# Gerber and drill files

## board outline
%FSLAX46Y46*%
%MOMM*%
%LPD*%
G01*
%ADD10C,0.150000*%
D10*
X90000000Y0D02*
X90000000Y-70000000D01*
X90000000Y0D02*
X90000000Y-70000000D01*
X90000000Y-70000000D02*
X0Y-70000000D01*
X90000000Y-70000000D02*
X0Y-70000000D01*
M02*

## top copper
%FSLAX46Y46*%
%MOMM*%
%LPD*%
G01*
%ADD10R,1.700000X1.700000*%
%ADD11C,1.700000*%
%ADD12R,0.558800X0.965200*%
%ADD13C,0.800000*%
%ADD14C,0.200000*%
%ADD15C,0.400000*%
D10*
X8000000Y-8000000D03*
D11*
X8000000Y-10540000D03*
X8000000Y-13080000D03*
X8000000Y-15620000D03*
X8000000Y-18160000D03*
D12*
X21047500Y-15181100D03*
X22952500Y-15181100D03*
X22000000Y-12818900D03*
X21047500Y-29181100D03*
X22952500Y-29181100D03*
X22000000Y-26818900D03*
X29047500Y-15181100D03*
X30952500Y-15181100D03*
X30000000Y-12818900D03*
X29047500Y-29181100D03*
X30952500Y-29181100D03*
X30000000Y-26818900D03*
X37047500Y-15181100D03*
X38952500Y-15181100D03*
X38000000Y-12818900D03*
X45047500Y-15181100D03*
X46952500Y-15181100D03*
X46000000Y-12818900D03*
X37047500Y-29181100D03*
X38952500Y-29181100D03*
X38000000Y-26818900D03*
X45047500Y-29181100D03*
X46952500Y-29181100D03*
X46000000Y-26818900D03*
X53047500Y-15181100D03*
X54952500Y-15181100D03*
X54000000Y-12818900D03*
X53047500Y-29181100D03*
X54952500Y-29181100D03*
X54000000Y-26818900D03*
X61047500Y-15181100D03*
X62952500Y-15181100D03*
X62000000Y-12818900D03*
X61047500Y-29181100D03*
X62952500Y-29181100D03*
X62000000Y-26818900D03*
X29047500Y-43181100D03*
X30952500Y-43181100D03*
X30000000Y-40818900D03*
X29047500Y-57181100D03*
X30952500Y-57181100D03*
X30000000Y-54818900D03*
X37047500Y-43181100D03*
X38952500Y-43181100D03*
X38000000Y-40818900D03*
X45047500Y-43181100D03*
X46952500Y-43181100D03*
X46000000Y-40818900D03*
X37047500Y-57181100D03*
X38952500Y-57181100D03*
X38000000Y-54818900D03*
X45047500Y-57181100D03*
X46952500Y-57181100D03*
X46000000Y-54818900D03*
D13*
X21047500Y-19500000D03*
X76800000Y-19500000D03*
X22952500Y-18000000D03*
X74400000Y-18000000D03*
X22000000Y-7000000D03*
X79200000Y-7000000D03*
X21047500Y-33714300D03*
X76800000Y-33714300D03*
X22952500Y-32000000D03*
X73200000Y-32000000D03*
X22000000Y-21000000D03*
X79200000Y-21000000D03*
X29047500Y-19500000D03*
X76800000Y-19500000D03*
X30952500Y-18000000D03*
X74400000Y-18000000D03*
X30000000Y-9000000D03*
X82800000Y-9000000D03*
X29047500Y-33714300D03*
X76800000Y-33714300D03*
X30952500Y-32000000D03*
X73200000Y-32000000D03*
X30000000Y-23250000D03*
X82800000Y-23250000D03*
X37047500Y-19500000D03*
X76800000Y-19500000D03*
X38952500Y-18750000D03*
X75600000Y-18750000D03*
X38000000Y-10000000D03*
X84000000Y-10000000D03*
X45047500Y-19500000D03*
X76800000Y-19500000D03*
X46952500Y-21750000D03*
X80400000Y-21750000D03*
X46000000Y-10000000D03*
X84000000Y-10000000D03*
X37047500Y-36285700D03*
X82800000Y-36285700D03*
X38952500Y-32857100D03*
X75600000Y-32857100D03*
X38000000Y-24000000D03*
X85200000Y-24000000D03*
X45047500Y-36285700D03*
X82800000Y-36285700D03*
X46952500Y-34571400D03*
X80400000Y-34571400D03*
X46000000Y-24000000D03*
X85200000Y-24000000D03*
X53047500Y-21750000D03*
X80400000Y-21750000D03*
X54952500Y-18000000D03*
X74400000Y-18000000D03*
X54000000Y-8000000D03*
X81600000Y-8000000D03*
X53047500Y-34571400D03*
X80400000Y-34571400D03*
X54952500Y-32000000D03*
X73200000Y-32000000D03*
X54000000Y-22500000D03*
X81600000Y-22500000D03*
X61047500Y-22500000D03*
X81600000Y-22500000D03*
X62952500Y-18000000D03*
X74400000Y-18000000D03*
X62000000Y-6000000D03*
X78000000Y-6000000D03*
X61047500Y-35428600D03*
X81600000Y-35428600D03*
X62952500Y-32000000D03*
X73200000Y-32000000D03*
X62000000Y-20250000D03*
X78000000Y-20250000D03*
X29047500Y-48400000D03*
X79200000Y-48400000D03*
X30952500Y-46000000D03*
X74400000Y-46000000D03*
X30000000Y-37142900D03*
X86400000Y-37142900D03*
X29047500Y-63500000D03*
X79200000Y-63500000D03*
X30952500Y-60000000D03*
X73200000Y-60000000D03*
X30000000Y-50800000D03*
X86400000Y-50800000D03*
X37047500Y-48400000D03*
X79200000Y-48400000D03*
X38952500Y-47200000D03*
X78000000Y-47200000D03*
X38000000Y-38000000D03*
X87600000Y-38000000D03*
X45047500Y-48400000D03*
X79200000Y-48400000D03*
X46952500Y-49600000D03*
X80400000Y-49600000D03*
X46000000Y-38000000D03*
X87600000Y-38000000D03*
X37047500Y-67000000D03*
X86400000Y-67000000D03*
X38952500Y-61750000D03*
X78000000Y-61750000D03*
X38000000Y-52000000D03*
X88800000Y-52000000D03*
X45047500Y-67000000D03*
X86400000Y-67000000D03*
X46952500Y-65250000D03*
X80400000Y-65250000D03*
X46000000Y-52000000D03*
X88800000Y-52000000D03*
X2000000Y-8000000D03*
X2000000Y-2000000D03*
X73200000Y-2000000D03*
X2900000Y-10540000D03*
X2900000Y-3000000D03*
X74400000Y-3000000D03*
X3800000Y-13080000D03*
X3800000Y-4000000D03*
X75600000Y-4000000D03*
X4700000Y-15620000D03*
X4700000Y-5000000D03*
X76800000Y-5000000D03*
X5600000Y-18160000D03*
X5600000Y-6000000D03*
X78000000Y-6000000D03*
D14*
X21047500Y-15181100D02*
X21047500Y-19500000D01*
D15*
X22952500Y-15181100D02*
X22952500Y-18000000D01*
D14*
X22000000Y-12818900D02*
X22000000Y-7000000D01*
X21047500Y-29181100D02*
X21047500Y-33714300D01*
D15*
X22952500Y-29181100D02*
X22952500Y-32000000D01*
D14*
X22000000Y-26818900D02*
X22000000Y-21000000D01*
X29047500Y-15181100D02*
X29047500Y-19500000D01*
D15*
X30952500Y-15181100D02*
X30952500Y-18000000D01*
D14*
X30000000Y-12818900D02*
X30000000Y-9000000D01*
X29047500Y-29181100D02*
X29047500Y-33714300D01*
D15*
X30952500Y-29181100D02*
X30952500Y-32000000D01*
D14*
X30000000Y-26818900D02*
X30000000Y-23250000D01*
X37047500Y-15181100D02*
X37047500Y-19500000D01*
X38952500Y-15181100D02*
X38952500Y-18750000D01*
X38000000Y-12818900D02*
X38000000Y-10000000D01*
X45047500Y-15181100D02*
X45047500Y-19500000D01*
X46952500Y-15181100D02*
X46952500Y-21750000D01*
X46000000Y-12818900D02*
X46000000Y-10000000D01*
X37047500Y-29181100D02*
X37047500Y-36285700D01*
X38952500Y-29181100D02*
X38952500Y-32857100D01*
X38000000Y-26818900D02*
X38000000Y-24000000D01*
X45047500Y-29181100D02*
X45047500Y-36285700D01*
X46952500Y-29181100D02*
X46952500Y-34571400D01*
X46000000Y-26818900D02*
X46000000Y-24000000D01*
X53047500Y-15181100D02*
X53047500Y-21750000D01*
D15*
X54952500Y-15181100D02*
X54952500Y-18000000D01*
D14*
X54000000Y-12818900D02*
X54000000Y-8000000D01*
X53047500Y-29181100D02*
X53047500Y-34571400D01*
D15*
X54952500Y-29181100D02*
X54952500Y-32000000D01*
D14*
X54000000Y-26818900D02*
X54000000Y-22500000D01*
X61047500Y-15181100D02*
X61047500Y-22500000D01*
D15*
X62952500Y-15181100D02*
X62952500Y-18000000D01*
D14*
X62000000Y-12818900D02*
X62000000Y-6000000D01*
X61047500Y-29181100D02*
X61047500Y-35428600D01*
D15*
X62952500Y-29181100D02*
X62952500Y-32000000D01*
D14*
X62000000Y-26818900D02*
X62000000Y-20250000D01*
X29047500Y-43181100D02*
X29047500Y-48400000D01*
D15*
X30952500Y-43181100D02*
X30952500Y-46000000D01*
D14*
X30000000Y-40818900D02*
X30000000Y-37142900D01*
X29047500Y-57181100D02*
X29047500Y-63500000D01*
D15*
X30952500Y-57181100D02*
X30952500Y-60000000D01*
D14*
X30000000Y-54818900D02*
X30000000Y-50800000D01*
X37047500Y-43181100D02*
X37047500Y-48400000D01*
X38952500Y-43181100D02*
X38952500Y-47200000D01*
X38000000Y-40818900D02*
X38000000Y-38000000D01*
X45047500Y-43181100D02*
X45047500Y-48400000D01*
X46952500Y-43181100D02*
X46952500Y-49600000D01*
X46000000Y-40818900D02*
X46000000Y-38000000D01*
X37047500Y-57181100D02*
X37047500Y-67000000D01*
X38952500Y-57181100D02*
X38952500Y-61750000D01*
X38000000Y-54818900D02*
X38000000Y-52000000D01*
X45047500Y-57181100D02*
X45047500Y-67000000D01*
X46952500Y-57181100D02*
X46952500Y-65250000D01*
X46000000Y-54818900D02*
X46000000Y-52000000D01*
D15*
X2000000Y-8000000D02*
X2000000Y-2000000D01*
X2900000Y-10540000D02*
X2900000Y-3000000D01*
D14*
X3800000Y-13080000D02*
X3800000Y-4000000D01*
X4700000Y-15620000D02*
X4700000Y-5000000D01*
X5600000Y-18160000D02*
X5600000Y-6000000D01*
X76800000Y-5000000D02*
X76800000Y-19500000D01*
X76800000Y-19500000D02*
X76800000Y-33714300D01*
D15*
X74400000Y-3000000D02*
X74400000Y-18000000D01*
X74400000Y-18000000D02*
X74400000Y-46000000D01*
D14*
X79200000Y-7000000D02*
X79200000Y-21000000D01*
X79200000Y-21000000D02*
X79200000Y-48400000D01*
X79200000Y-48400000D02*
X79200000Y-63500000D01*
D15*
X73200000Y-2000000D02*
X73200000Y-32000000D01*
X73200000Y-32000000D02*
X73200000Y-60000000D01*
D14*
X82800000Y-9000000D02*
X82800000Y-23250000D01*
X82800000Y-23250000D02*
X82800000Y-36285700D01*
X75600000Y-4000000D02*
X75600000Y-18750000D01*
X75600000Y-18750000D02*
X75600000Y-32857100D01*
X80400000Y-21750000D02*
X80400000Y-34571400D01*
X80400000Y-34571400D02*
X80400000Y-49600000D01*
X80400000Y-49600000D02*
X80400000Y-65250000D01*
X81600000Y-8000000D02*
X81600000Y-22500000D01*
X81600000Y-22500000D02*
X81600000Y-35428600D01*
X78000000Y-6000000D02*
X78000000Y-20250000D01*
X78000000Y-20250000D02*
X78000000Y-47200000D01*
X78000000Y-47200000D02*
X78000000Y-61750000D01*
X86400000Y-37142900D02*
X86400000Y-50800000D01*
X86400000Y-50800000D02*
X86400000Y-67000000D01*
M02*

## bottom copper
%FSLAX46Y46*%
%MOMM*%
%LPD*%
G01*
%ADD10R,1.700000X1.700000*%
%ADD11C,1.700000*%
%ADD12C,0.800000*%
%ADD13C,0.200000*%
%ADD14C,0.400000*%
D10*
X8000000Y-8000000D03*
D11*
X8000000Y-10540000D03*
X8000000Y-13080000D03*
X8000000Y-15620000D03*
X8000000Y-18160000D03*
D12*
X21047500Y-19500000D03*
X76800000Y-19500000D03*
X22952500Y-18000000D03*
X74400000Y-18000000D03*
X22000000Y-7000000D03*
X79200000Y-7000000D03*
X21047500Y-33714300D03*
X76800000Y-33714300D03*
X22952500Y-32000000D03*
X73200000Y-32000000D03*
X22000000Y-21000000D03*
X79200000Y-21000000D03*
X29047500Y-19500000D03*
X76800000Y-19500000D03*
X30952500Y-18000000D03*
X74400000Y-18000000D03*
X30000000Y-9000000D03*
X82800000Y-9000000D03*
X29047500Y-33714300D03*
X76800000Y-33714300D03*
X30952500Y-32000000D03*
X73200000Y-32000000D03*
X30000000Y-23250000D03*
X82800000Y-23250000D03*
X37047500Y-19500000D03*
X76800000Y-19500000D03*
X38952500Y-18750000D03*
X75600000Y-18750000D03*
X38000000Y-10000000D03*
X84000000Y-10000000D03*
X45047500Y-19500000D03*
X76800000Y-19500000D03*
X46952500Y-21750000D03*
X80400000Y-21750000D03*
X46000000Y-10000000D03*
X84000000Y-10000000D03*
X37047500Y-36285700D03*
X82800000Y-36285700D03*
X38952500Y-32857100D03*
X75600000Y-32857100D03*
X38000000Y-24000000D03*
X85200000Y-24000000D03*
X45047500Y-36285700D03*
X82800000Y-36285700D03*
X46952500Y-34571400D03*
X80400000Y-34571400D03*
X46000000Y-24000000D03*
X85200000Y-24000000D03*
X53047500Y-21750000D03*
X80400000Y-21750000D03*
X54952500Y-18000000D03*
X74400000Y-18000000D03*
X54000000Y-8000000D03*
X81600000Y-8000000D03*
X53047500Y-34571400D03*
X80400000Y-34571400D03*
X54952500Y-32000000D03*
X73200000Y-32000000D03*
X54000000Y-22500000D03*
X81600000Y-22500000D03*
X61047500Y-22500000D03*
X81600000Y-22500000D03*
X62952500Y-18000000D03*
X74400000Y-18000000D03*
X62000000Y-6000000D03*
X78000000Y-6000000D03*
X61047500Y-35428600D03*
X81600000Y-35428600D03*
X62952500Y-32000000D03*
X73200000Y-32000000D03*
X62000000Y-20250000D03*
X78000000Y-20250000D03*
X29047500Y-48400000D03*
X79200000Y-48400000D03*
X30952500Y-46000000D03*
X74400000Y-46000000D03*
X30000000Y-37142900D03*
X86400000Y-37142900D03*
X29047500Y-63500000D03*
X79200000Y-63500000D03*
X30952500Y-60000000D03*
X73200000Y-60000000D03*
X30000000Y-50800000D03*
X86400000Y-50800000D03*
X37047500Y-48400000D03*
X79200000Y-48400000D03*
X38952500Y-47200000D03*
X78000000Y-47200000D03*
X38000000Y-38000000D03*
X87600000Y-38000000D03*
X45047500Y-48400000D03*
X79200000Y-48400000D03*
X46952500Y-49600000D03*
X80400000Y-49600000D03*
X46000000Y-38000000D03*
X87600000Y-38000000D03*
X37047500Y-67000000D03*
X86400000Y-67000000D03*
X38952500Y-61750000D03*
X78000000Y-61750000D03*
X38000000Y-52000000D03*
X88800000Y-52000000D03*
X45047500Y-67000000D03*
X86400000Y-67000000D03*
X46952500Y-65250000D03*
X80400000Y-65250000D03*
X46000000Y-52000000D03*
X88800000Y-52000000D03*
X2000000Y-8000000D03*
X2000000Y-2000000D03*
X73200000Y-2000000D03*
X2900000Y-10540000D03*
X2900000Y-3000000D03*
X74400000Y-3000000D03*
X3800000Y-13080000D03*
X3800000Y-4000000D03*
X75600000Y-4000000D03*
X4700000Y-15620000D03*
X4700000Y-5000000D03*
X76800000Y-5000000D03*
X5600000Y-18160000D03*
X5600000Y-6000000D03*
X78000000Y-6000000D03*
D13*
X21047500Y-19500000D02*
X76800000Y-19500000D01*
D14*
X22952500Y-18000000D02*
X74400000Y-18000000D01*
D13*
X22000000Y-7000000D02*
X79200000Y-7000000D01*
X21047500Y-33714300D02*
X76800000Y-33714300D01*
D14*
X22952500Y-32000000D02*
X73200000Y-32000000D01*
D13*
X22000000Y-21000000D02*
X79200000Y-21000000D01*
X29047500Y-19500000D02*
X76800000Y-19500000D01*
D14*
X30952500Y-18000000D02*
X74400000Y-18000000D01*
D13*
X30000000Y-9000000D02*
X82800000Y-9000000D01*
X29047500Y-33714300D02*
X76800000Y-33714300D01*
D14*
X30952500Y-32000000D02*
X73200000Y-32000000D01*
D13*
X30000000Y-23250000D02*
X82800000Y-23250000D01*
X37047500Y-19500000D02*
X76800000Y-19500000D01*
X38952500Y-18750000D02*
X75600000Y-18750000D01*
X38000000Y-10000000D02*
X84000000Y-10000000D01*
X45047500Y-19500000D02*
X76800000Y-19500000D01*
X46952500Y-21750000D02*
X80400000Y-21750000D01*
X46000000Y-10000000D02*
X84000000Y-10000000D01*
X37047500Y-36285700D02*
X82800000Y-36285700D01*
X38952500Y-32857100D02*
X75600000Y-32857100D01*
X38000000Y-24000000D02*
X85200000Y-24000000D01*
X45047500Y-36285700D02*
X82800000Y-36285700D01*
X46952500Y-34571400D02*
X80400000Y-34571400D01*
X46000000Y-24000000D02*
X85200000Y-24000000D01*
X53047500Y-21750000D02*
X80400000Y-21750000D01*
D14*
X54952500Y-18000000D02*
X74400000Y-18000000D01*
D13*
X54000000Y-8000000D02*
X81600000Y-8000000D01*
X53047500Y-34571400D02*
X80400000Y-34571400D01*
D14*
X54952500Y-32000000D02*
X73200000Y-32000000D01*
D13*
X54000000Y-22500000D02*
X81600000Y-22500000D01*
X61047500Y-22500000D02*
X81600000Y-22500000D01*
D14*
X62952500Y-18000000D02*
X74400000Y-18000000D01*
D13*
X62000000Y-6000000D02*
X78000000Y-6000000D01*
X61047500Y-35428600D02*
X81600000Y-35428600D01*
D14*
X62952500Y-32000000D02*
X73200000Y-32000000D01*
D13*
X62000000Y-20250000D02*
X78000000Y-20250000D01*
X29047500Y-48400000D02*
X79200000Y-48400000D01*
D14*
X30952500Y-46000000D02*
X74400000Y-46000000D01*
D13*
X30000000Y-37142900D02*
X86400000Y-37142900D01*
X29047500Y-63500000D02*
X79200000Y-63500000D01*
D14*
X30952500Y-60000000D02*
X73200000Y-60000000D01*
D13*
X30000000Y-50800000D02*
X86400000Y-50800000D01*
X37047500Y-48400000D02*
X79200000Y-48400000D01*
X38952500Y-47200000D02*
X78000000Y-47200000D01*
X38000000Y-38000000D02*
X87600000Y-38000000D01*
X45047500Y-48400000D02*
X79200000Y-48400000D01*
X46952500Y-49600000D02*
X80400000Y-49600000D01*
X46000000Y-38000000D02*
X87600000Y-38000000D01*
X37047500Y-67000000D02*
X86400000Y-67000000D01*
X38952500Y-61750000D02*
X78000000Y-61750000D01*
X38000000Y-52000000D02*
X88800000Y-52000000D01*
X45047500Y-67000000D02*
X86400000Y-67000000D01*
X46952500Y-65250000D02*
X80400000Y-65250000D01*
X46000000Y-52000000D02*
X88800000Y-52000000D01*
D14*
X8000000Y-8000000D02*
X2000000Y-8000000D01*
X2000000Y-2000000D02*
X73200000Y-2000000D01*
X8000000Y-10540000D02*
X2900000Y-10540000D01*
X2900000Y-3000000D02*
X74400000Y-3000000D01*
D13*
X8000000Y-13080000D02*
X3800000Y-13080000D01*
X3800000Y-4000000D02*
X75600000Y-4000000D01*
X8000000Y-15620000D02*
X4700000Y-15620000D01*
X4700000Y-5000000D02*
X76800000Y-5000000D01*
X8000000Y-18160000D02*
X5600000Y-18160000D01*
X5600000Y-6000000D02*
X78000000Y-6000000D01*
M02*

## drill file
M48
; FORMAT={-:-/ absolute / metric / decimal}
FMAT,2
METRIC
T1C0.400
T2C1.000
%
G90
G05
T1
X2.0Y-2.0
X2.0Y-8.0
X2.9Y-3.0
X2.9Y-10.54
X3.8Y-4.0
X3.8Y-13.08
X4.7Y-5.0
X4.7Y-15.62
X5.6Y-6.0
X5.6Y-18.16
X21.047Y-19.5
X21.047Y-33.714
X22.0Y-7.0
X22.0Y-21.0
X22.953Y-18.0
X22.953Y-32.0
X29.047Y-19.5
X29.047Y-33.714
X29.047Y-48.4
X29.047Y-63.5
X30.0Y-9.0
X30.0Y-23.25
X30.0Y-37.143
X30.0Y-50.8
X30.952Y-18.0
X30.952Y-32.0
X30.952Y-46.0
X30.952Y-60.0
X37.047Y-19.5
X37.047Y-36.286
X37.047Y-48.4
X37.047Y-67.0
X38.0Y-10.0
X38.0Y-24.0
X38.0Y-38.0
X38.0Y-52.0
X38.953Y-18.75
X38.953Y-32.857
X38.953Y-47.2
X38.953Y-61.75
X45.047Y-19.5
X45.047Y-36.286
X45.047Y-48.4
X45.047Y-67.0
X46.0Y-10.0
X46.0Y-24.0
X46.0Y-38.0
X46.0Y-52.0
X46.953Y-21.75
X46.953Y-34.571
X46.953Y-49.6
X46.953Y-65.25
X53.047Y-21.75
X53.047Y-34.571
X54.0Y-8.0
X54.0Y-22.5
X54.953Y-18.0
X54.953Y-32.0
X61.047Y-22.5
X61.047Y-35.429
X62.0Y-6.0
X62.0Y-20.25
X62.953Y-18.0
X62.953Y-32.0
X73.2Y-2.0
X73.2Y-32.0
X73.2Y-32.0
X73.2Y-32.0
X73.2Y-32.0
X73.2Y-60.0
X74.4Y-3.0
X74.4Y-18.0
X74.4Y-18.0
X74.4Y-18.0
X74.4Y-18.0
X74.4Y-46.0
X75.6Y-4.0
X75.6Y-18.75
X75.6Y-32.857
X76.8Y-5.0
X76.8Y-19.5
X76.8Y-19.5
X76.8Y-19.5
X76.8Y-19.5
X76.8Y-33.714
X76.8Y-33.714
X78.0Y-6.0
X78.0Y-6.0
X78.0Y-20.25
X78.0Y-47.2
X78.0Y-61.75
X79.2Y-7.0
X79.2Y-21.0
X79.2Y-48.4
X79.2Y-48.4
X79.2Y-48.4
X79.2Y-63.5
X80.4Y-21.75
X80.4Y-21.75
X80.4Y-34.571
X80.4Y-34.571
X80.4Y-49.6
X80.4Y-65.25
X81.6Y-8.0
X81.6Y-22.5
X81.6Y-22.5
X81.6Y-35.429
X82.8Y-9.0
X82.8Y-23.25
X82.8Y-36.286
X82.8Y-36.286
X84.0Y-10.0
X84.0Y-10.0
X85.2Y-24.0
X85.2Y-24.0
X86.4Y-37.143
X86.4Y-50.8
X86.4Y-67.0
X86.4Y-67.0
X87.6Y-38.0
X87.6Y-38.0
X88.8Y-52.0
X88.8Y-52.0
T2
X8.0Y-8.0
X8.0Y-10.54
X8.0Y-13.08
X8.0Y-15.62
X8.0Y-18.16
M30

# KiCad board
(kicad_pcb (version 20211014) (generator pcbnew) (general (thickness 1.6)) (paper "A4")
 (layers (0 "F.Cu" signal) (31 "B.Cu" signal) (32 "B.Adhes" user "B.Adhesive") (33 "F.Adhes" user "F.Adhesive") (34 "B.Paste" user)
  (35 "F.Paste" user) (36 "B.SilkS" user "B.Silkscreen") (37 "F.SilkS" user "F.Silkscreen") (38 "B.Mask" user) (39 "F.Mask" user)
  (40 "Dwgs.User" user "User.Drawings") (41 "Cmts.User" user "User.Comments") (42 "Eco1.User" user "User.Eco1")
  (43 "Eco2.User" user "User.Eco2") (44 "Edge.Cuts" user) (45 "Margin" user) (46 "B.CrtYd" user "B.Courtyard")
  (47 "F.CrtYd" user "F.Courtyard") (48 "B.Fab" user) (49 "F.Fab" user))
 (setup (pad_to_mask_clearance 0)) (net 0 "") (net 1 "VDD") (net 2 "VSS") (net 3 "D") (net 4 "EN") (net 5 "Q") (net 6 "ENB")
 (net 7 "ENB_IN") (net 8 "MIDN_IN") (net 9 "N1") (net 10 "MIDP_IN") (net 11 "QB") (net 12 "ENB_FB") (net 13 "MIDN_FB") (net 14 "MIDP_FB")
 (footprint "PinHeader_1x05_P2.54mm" (layer "F.Cu") (at 8.0 8.0)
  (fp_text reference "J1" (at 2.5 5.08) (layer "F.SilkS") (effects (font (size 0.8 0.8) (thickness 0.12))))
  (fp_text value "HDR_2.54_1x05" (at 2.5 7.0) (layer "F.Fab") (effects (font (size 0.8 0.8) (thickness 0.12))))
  (pad "1" thru_hole rect (at 0 0.0) (size 1.7 1.7) (drill 1.0) (layers *.Cu *.Mask) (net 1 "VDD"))
  (pad "2" thru_hole circle (at 0 2.54) (size 1.7 1.7) (drill 1.0) (layers *.Cu *.Mask) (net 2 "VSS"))
  (pad "3" thru_hole circle (at 0 5.08) (size 1.7 1.7) (drill 1.0) (layers *.Cu *.Mask) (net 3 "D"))
  (pad "4" thru_hole circle (at 0 7.62) (size 1.7 1.7) (drill 1.0) (layers *.Cu *.Mask) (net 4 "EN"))
  (pad "5" thru_hole circle (at 0 10.16) (size 1.7 1.7) (drill 1.0) (layers *.Cu *.Mask) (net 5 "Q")))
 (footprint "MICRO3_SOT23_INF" (layer "F.Cu") (at 22.0000 14.0000)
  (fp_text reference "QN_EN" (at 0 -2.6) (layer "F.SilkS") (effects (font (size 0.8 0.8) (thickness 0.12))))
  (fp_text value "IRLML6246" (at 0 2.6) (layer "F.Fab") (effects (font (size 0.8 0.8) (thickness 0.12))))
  (pad "1" smd rect (at -0.9525 1.1811) (size 0.5588 0.9652) (layers "F.Cu" "F.Paste" "F.Mask") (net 4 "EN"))
  (pad "2" smd rect (at 0.9525 1.1811) (size 0.5588 0.9652) (layers "F.Cu" "F.Paste" "F.Mask") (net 2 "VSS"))
  (pad "3" smd rect (at 0 -1.1811) (size 0.5588 0.9652) (layers "F.Cu" "F.Paste" "F.Mask") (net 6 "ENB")))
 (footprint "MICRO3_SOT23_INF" (layer "F.Cu") (at 22.0000 28.0000)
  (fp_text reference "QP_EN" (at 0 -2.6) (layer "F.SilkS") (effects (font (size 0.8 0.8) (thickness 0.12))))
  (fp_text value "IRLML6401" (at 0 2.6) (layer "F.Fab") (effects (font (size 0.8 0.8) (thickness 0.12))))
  (pad "1" smd rect (at -0.9525 1.1811) (size 0.5588 0.9652) (layers "F.Cu" "F.Paste" "F.Mask") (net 4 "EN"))
  (pad "2" smd rect (at 0.9525 1.1811) (size 0.5588 0.9652) (layers "F.Cu" "F.Paste" "F.Mask") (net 1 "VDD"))
  (pad "3" smd rect (at 0 -1.1811) (size 0.5588 0.9652) (layers "F.Cu" "F.Paste" "F.Mask") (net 6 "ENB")))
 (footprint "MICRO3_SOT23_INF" (layer "F.Cu") (at 30.0000 14.0000)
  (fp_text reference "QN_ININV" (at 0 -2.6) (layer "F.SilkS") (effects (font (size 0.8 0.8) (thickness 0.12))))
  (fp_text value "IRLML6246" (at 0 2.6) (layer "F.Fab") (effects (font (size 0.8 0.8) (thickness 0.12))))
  (pad "1" smd rect (at -0.9525 1.1811) (size 0.5588 0.9652) (layers "F.Cu" "F.Paste" "F.Mask") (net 4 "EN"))
  (pad "2" smd rect (at 0.9525 1.1811) (size 0.5588 0.9652) (layers "F.Cu" "F.Paste" "F.Mask") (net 2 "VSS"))
  (pad "3" smd rect (at 0 -1.1811) (size 0.5588 0.9652) (layers "F.Cu" "F.Paste" "F.Mask") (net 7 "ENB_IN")))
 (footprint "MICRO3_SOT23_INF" (layer "F.Cu") (at 30.0000 28.0000)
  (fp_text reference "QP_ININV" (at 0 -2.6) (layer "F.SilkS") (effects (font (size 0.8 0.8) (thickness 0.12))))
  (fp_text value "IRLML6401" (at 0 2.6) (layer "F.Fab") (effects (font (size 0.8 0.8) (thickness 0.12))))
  (pad "1" smd rect (at -0.9525 1.1811) (size 0.5588 0.9652) (layers "F.Cu" "F.Paste" "F.Mask") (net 4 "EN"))
  (pad "2" smd rect (at 0.9525 1.1811) (size 0.5588 0.9652) (layers "F.Cu" "F.Paste" "F.Mask") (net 1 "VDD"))
  (pad "3" smd rect (at 0 -1.1811) (size 0.5588 0.9652) (layers "F.Cu" "F.Paste" "F.Mask") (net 7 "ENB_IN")))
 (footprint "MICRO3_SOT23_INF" (layer "F.Cu") (at 38.0000 14.0000)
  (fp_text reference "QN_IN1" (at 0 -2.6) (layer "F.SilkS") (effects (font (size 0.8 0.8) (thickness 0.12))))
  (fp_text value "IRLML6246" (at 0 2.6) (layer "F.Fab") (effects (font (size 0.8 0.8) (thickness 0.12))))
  (pad "1" smd rect (at -0.9525 1.1811) (size 0.5588 0.9652) (layers "F.Cu" "F.Paste" "F.Mask") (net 4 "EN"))
  (pad "2" smd rect (at 0.9525 1.1811) (size 0.5588 0.9652) (layers "F.Cu" "F.Paste" "F.Mask") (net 3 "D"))
  (pad "3" smd rect (at 0 -1.1811) (size 0.5588 0.9652) (layers "F.Cu" "F.Paste" "F.Mask") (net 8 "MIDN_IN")))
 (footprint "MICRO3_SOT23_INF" (layer "F.Cu") (at 46.0000 14.0000)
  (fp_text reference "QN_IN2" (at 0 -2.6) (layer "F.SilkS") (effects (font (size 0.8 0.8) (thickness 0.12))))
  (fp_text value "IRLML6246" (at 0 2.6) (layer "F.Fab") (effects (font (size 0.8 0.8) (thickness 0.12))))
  (pad "1" smd rect (at -0.9525 1.1811) (size 0.5588 0.9652) (layers "F.Cu" "F.Paste" "F.Mask") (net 4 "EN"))
  (pad "2" smd rect (at 0.9525 1.1811) (size 0.5588 0.9652) (layers "F.Cu" "F.Paste" "F.Mask") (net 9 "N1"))
  (pad "3" smd rect (at 0 -1.1811) (size 0.5588 0.9652) (layers "F.Cu" "F.Paste" "F.Mask") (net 8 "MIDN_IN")))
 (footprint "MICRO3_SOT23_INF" (layer "F.Cu") (at 38.0000 28.0000)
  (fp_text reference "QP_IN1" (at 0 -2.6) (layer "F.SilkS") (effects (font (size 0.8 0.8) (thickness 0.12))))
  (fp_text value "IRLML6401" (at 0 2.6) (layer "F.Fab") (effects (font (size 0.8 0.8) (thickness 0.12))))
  (pad "1" smd rect (at -0.9525 1.1811) (size 0.5588 0.9652) (layers "F.Cu" "F.Paste" "F.Mask") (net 7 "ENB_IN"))
  (pad "2" smd rect (at 0.9525 1.1811) (size 0.5588 0.9652) (layers "F.Cu" "F.Paste" "F.Mask") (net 3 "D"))
  (pad "3" smd rect (at 0 -1.1811) (size 0.5588 0.9652) (layers "F.Cu" "F.Paste" "F.Mask") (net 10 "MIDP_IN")))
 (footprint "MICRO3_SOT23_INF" (layer "F.Cu") (at 46.0000 28.0000)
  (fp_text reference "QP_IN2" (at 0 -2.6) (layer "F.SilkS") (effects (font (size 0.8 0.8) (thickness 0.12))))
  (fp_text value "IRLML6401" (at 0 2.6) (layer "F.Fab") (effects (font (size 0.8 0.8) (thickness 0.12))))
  (pad "1" smd rect (at -0.9525 1.1811) (size 0.5588 0.9652) (layers "F.Cu" "F.Paste" "F.Mask") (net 7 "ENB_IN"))
  (pad "2" smd rect (at 0.9525 1.1811) (size 0.5588 0.9652) (layers "F.Cu" "F.Paste" "F.Mask") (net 9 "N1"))
  (pad "3" smd rect (at 0 -1.1811) (size 0.5588 0.9652) (layers "F.Cu" "F.Paste" "F.Mask") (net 10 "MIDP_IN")))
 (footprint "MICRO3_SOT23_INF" (layer "F.Cu") (at 54.0000 14.0000)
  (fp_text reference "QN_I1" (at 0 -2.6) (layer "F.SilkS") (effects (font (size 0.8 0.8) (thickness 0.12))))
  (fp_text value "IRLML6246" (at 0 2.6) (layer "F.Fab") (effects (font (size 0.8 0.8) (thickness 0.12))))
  (pad "1" smd rect (at -0.9525 1.1811) (size 0.5588 0.9652) (layers "F.Cu" "F.Paste" "F.Mask") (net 9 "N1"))
  (pad "2" smd rect (at 0.9525 1.1811) (size 0.5588 0.9652) (layers "F.Cu" "F.Paste" "F.Mask") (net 2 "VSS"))
  (pad "3" smd rect (at 0 -1.1811) (size 0.5588 0.9652) (layers "F.Cu" "F.Paste" "F.Mask") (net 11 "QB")))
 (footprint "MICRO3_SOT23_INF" (layer "F.Cu") (at 54.0000 28.0000)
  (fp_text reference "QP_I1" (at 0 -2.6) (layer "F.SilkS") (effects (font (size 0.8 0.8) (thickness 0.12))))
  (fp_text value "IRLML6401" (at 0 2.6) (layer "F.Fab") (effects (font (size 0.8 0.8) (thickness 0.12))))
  (pad "1" smd rect (at -0.9525 1.1811) (size 0.5588 0.9652) (layers "F.Cu" "F.Paste" "F.Mask") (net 9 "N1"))
  (pad "2" smd rect (at 0.9525 1.1811) (size 0.5588 0.9652) (layers "F.Cu" "F.Paste" "F.Mask") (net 1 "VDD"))
  (pad "3" smd rect (at 0 -1.1811) (size 0.5588 0.9652) (layers "F.Cu" "F.Paste" "F.Mask") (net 11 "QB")))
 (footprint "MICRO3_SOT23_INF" (layer "F.Cu") (at 62.0000 14.0000)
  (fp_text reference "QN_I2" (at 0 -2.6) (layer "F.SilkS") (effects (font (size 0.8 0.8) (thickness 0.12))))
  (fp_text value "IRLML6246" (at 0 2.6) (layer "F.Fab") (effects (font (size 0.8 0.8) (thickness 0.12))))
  (pad "1" smd rect (at -0.9525 1.1811) (size 0.5588 0.9652) (layers "F.Cu" "F.Paste" "F.Mask") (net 11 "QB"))
  (pad "2" smd rect (at 0.9525 1.1811) (size 0.5588 0.9652) (layers "F.Cu" "F.Paste" "F.Mask") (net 2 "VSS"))
  (pad "3" smd rect (at 0 -1.1811) (size 0.5588 0.9652) (layers "F.Cu" "F.Paste" "F.Mask") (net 5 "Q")))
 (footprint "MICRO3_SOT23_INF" (layer "F.Cu") (at 62.0000 28.0000)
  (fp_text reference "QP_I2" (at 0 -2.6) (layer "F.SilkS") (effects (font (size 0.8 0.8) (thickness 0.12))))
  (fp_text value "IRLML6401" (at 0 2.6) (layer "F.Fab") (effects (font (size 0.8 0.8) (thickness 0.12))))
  (pad "1" smd rect (at -0.9525 1.1811) (size 0.5588 0.9652) (layers "F.Cu" "F.Paste" "F.Mask") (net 11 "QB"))
  (pad "2" smd rect (at 0.9525 1.1811) (size 0.5588 0.9652) (layers "F.Cu" "F.Paste" "F.Mask") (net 1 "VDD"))
  (pad "3" smd rect (at 0 -1.1811) (size 0.5588 0.9652) (layers "F.Cu" "F.Paste" "F.Mask") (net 5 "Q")))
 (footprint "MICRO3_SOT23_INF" (layer "F.Cu") (at 30.0000 42.0000)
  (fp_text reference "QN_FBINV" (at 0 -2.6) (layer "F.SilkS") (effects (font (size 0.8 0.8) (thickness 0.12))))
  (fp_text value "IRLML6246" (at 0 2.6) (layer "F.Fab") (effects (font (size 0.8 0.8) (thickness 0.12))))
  (pad "1" smd rect (at -0.9525 1.1811) (size 0.5588 0.9652) (layers "F.Cu" "F.Paste" "F.Mask") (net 6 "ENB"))
  (pad "2" smd rect (at 0.9525 1.1811) (size 0.5588 0.9652) (layers "F.Cu" "F.Paste" "F.Mask") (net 2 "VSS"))
  (pad "3" smd rect (at 0 -1.1811) (size 0.5588 0.9652) (layers "F.Cu" "F.Paste" "F.Mask") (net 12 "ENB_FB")))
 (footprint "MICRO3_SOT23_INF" (layer "F.Cu") (at 30.0000 56.0000)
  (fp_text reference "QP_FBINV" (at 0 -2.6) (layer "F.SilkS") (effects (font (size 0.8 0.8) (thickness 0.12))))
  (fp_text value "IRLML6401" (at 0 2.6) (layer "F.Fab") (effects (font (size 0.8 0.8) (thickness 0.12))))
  (pad "1" smd rect (at -0.9525 1.1811) (size 0.5588 0.9652) (layers "F.Cu" "F.Paste" "F.Mask") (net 6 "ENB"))
  (pad "2" smd rect (at 0.9525 1.1811) (size 0.5588 0.9652) (layers "F.Cu" "F.Paste" "F.Mask") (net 1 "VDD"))
  (pad "3" smd rect (at 0 -1.1811) (size 0.5588 0.9652) (layers "F.Cu" "F.Paste" "F.Mask") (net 12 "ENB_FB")))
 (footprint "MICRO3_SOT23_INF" (layer "F.Cu") (at 38.0000 42.0000)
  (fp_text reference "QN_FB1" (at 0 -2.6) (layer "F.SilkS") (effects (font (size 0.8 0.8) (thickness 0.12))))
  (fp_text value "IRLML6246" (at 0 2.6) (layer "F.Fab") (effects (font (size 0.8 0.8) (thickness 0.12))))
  (pad "1" smd rect (at -0.9525 1.1811) (size 0.5588 0.9652) (layers "F.Cu" "F.Paste" "F.Mask") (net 6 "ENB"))
  (pad "2" smd rect (at 0.9525 1.1811) (size 0.5588 0.9652) (layers "F.Cu" "F.Paste" "F.Mask") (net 5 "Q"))
  (pad "3" smd rect (at 0 -1.1811) (size 0.5588 0.9652) (layers "F.Cu" "F.Paste" "F.Mask") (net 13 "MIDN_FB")))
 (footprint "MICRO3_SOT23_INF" (layer "F.Cu") (at 46.0000 42.0000)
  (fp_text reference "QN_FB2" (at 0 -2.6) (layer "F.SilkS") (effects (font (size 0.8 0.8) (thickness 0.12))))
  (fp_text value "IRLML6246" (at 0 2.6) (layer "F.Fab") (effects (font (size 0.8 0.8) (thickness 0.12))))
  (pad "1" smd rect (at -0.9525 1.1811) (size 0.5588 0.9652) (layers "F.Cu" "F.Paste" "F.Mask") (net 6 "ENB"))
  (pad "2" smd rect (at 0.9525 1.1811) (size 0.5588 0.9652) (layers "F.Cu" "F.Paste" "F.Mask") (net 9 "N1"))
  (pad "3" smd rect (at 0 -1.1811) (size 0.5588 0.9652) (layers "F.Cu" "F.Paste" "F.Mask") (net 13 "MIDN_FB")))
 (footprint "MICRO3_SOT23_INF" (layer "F.Cu") (at 38.0000 56.0000)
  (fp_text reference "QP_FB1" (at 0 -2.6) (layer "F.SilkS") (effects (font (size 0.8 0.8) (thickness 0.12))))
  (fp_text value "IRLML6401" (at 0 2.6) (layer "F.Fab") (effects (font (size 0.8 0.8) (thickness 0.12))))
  (pad "1" smd rect (at -0.9525 1.1811) (size 0.5588 0.9652) (layers "F.Cu" "F.Paste" "F.Mask") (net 12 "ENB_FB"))
  (pad "2" smd rect (at 0.9525 1.1811) (size 0.5588 0.9652) (layers "F.Cu" "F.Paste" "F.Mask") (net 5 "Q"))
  (pad "3" smd rect (at 0 -1.1811) (size 0.5588 0.9652) (layers "F.Cu" "F.Paste" "F.Mask") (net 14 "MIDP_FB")))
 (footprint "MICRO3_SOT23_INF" (layer "F.Cu") (at 46.0000 56.0000)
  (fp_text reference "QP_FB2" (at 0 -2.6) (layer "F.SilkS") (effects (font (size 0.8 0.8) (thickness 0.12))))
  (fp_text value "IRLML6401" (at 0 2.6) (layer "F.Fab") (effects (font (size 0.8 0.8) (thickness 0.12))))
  (pad "1" smd rect (at -0.9525 1.1811) (size 0.5588 0.9652) (layers "F.Cu" "F.Paste" "F.Mask") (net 12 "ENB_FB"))
  (pad "2" smd rect (at 0.9525 1.1811) (size 0.5588 0.9652) (layers "F.Cu" "F.Paste" "F.Mask") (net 9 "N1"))
  (pad "3" smd rect (at 0 -1.1811) (size 0.5588 0.9652) (layers "F.Cu" "F.Paste" "F.Mask") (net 14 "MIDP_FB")))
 (gr_line (start 90 0) (end 90 70) (layer "Edge.Cuts") (width 0.15))
 (gr_line (start 90 0) (end 90 70) (layer "Edge.Cuts") (width 0.15))
 (gr_line (start 90 70) (end 0 70) (layer "Edge.Cuts") (width 0.15))
 (gr_line (start 90 70) (end 0 70) (layer "Edge.Cuts") (width 0.15))
 (segment (start 21.0475 15.1811) (end 21.0475 19.5) (width 0.2) (layer "F.Cu") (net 4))
 (segment (start 21.0475 19.5) (end 76.8 19.5) (width 0.2) (layer "B.Cu") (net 4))
 (segment (start 22.9525 15.1811) (end 22.9525 18.0) (width 0.4) (layer "F.Cu") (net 2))
 (segment (start 22.9525 18.0) (end 74.4 18.0) (width 0.4) (layer "B.Cu") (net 2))
 (segment (start 22.0 12.8189) (end 22.0 7.0) (width 0.2) (layer "F.Cu") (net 6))
 (segment (start 22.0 7.0) (end 79.2 7.0) (width 0.2) (layer "B.Cu") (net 6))
 (segment (start 21.0475 29.1811) (end 21.0475 33.7143) (width 0.2) (layer "F.Cu") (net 4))
 (segment (start 21.0475 33.7143) (end 76.8 33.7143) (width 0.2) (layer "B.Cu") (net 4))
 (segment (start 22.9525 29.1811) (end 22.9525 32.0) (width 0.4) (layer "F.Cu") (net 1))
 (segment (start 22.9525 32.0) (end 73.2 32.0) (width 0.4) (layer "B.Cu") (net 1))
 (segment (start 22.0 26.8189) (end 22.0 21.0) (width 0.2) (layer "F.Cu") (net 6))
 (segment (start 22.0 21.0) (end 79.2 21.0) (width 0.2) (layer "B.Cu") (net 6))
 (segment (start 29.0475 15.1811) (end 29.0475 19.5) (width 0.2) (layer "F.Cu") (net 4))
 (segment (start 29.0475 19.5) (end 76.8 19.5) (width 0.2) (layer "B.Cu") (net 4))
 (segment (start 30.9525 15.1811) (end 30.9525 18.0) (width 0.4) (layer "F.Cu") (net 2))
 (segment (start 30.9525 18.0) (end 74.4 18.0) (width 0.4) (layer "B.Cu") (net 2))
 (segment (start 30.0 12.8189) (end 30.0 9.0) (width 0.2) (layer "F.Cu") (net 7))
 (segment (start 30.0 9.0) (end 82.8 9.0) (width 0.2) (layer "B.Cu") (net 7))
 (segment (start 29.0475 29.1811) (end 29.0475 33.7143) (width 0.2) (layer "F.Cu") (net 4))
 (segment (start 29.0475 33.7143) (end 76.8 33.7143) (width 0.2) (layer "B.Cu") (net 4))
 (segment (start 30.9525 29.1811) (end 30.9525 32.0) (width 0.4) (layer "F.Cu") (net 1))
 (segment (start 30.9525 32.0) (end 73.2 32.0) (width 0.4) (layer "B.Cu") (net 1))
 (segment (start 30.0 26.8189) (end 30.0 23.25) (width 0.2) (layer "F.Cu") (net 7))
 (segment (start 30.0 23.25) (end 82.8 23.25) (width 0.2) (layer "B.Cu") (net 7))
 (segment (start 37.0475 15.1811) (end 37.0475 19.5) (width 0.2) (layer "F.Cu") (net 4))
 (segment (start 37.0475 19.5) (end 76.8 19.5) (width 0.2) (layer "B.Cu") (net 4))
 (segment (start 38.9525 15.1811) (end 38.9525 18.75) (width 0.2) (layer "F.Cu") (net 3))
 (segment (start 38.9525 18.75) (end 75.6 18.75) (width 0.2) (layer "B.Cu") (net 3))
 (segment (start 38.0 12.8189) (end 38.0 10.0) (width 0.2) (layer "F.Cu") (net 8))
 (segment (start 38.0 10.0) (end 84.0 10.0) (width 0.2) (layer "B.Cu") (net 8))
 (segment (start 45.0475 15.1811) (end 45.0475 19.5) (width 0.2) (layer "F.Cu") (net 4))
 (segment (start 45.0475 19.5) (end 76.8 19.5) (width 0.2) (layer "B.Cu") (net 4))
 (segment (start 46.9525 15.1811) (end 46.9525 21.75) (width 0.2) (layer "F.Cu") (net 9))
 (segment (start 46.9525 21.75) (end 80.4 21.75) (width 0.2) (layer "B.Cu") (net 9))
 (segment (start 46.0 12.8189) (end 46.0 10.0) (width 0.2) (layer "F.Cu") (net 8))
 (segment (start 46.0 10.0) (end 84.0 10.0) (width 0.2) (layer "B.Cu") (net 8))
 (segment (start 37.0475 29.1811) (end 37.0475 36.2857) (width 0.2) (layer "F.Cu") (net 7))
 (segment (start 37.0475 36.2857) (end 82.8 36.2857) (width 0.2) (layer "B.Cu") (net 7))
 (segment (start 38.9525 29.1811) (end 38.9525 32.8571) (width 0.2) (layer "F.Cu") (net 3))
 (segment (start 38.9525 32.8571) (end 75.6 32.8571) (width 0.2) (layer "B.Cu") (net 3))
 (segment (start 38.0 26.8189) (end 38.0 24.0) (width 0.2) (layer "F.Cu") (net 10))
 (segment (start 38.0 24.0) (end 85.2 24.0) (width 0.2) (layer "B.Cu") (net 10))
 (segment (start 45.0475 29.1811) (end 45.0475 36.2857) (width 0.2) (layer "F.Cu") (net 7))
 (segment (start 45.0475 36.2857) (end 82.8 36.2857) (width 0.2) (layer "B.Cu") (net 7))
 (segment (start 46.9525 29.1811) (end 46.9525 34.5714) (width 0.2) (layer "F.Cu") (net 9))
 (segment (start 46.9525 34.5714) (end 80.4 34.5714) (width 0.2) (layer "B.Cu") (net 9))
 (segment (start 46.0 26.8189) (end 46.0 24.0) (width 0.2) (layer "F.Cu") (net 10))
 (segment (start 46.0 24.0) (end 85.2 24.0) (width 0.2) (layer "B.Cu") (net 10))
 (segment (start 53.0475 15.1811) (end 53.0475 21.75) (width 0.2) (layer "F.Cu") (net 9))
 (segment (start 53.0475 21.75) (end 80.4 21.75) (width 0.2) (layer "B.Cu") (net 9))
 (segment (start 54.9525 15.1811) (end 54.9525 18.0) (width 0.4) (layer "F.Cu") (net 2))
 (segment (start 54.9525 18.0) (end 74.4 18.0) (width 0.4) (layer "B.Cu") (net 2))
 (segment (start 54.0 12.8189) (end 54.0 8.0) (width 0.2) (layer "F.Cu") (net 11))
 (segment (start 54.0 8.0) (end 81.6 8.0) (width 0.2) (layer "B.Cu") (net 11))
 (segment (start 53.0475 29.1811) (end 53.0475 34.5714) (width 0.2) (layer "F.Cu") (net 9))
 (segment (start 53.0475 34.5714) (end 80.4 34.5714) (width 0.2) (layer "B.Cu") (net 9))
 (segment (start 54.9525 29.1811) (end 54.9525 32.0) (width 0.4) (layer "F.Cu") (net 1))
 (segment (start 54.9525 32.0) (end 73.2 32.0) (width 0.4) (layer "B.Cu") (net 1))
 (segment (start 54.0 26.8189) (end 54.0 22.5) (width 0.2) (layer "F.Cu") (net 11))
 (segment (start 54.0 22.5) (end 81.6 22.5) (width 0.2) (layer "B.Cu") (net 11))
 (segment (start 61.0475 15.1811) (end 61.0475 22.5) (width 0.2) (layer "F.Cu") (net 11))
 (segment (start 61.0475 22.5) (end 81.6 22.5) (width 0.2) (layer "B.Cu") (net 11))
 (segment (start 62.9525 15.1811) (end 62.9525 18.0) (width 0.4) (layer "F.Cu") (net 2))
 (segment (start 62.9525 18.0) (end 74.4 18.0) (width 0.4) (layer "B.Cu") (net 2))
 (segment (start 62.0 12.8189) (end 62.0 6.0) (width 0.2) (layer "F.Cu") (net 5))
 (segment (start 62.0 6.0) (end 78.0 6.0) (width 0.2) (layer "B.Cu") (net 5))
 (segment (start 61.0475 29.1811) (end 61.0475 35.4286) (width 0.2) (layer "F.Cu") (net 11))
 (segment (start 61.0475 35.4286) (end 81.6 35.4286) (width 0.2) (layer "B.Cu") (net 11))
 (segment (start 62.9525 29.1811) (end 62.9525 32.0) (width 0.4) (layer "F.Cu") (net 1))
 (segment (start 62.9525 32.0) (end 73.2 32.0) (width 0.4) (layer "B.Cu") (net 1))
 (segment (start 62.0 26.8189) (end 62.0 20.25) (width 0.2) (layer "F.Cu") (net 5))
 (segment (start 62.0 20.25) (end 78.0 20.25) (width 0.2) (layer "B.Cu") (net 5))
 (segment (start 29.0475 43.1811) (end 29.0475 48.4) (width 0.2) (layer "F.Cu") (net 6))
 (segment (start 29.0475 48.4) (end 79.2 48.4) (width 0.2) (layer "B.Cu") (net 6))
 (segment (start 30.9525 43.1811) (end 30.9525 46.0) (width 0.4) (layer "F.Cu") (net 2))
 (segment (start 30.9525 46.0) (end 74.4 46.0) (width 0.4) (layer "B.Cu") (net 2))
 (segment (start 30.0 40.8189) (end 30.0 37.1429) (width 0.2) (layer "F.Cu") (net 12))
 (segment (start 30.0 37.1429) (end 86.4 37.1429) (width 0.2) (layer "B.Cu") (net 12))
 (segment (start 29.0475 57.1811) (end 29.0475 63.5) (width 0.2) (layer "F.Cu") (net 6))
 (segment (start 29.0475 63.5) (end 79.2 63.5) (width 0.2) (layer "B.Cu") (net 6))
 (segment (start 30.9525 57.1811) (end 30.9525 60.0) (width 0.4) (layer "F.Cu") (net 1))
 (segment (start 30.9525 60.0) (end 73.2 60.0) (width 0.4) (layer "B.Cu") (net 1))
 (segment (start 30.0 54.8189) (end 30.0 50.8) (width 0.2) (layer "F.Cu") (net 12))
 (segment (start 30.0 50.8) (end 86.4 50.8) (width 0.2) (layer "B.Cu") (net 12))
 (segment (start 37.0475 43.1811) (end 37.0475 48.4) (width 0.2) (layer "F.Cu") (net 6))
 (segment (start 37.0475 48.4) (end 79.2 48.4) (width 0.2) (layer "B.Cu") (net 6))
 (segment (start 38.9525 43.1811) (end 38.9525 47.2) (width 0.2) (layer "F.Cu") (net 5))
 (segment (start 38.9525 47.2) (end 78.0 47.2) (width 0.2) (layer "B.Cu") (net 5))
 (segment (start 38.0 40.8189) (end 38.0 38.0) (width 0.2) (layer "F.Cu") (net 13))
 (segment (start 38.0 38.0) (end 87.6 38.0) (width 0.2) (layer "B.Cu") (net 13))
 (segment (start 45.0475 43.1811) (end 45.0475 48.4) (width 0.2) (layer "F.Cu") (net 6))
 (segment (start 45.0475 48.4) (end 79.2 48.4) (width 0.2) (layer "B.Cu") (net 6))
 (segment (start 46.9525 43.1811) (end 46.9525 49.6) (width 0.2) (layer "F.Cu") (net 9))
 (segment (start 46.9525 49.6) (end 80.4 49.6) (width 0.2) (layer "B.Cu") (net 9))
 (segment (start 46.0 40.8189) (end 46.0 38.0) (width 0.2) (layer "F.Cu") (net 13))
 (segment (start 46.0 38.0) (end 87.6 38.0) (width 0.2) (layer "B.Cu") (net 13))
 (segment (start 37.0475 57.1811) (end 37.0475 67.0) (width 0.2) (layer "F.Cu") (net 12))
 (segment (start 37.0475 67.0) (end 86.4 67.0) (width 0.2) (layer "B.Cu") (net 12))
 (segment (start 38.9525 57.1811) (end 38.9525 61.75) (width 0.2) (layer "F.Cu") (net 5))
 (segment (start 38.9525 61.75) (end 78.0 61.75) (width 0.2) (layer "B.Cu") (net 5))
 (segment (start 38.0 54.8189) (end 38.0 52.0) (width 0.2) (layer "F.Cu") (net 14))
 (segment (start 38.0 52.0) (end 88.8 52.0) (width 0.2) (layer "B.Cu") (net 14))
 (segment (start 45.0475 57.1811) (end 45.0475 67.0) (width 0.2) (layer "F.Cu") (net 12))
 (segment (start 45.0475 67.0) (end 86.4 67.0) (width 0.2) (layer "B.Cu") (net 12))
 (segment (start 46.9525 57.1811) (end 46.9525 65.25) (width 0.2) (layer "F.Cu") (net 9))
 (segment (start 46.9525 65.25) (end 80.4 65.25) (width 0.2) (layer "B.Cu") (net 9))
 (segment (start 46.0 54.8189) (end 46.0 52.0) (width 0.2) (layer "F.Cu") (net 14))
 (segment (start 46.0 52.0) (end 88.8 52.0) (width 0.2) (layer "B.Cu") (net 14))
 (segment (start 8.0 8.0) (end 2.0 8.0) (width 0.4) (layer "B.Cu") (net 1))
 (segment (start 2.0 8.0) (end 2.0 2.0) (width 0.4) (layer "F.Cu") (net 1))
 (segment (start 2.0 2.0) (end 73.2 2.0) (width 0.4) (layer "B.Cu") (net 1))
 (segment (start 8.0 10.54) (end 2.9 10.54) (width 0.4) (layer "B.Cu") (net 2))
 (segment (start 2.9 10.54) (end 2.9 3.0) (width 0.4) (layer "F.Cu") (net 2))
 (segment (start 2.9 3.0) (end 74.4 3.0) (width 0.4) (layer "B.Cu") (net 2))
 (segment (start 8.0 13.08) (end 3.8 13.08) (width 0.2) (layer "B.Cu") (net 3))
 (segment (start 3.8 13.08) (end 3.8 4.0) (width 0.2) (layer "F.Cu") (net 3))
 (segment (start 3.8 4.0) (end 75.6 4.0) (width 0.2) (layer "B.Cu") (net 3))
 (segment (start 8.0 15.62) (end 4.7 15.62) (width 0.2) (layer "B.Cu") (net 4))
 (segment (start 4.7 15.62) (end 4.7 5.0) (width 0.2) (layer "F.Cu") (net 4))
 (segment (start 4.7 5.0) (end 76.8 5.0) (width 0.2) (layer "B.Cu") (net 4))
 (segment (start 8.0 18.16) (end 5.6 18.16) (width 0.2) (layer "B.Cu") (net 5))
 (segment (start 5.6 18.16) (end 5.6 6.0) (width 0.2) (layer "F.Cu") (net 5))
 (segment (start 5.6 6.0) (end 78.0 6.0) (width 0.2) (layer "B.Cu") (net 5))
 (segment (start 76.8 5.0) (end 76.8 19.5) (width 0.2) (layer "F.Cu") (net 4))
 (segment (start 76.8 19.5) (end 76.8 33.7143) (width 0.2) (layer "F.Cu") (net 4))
 (segment (start 74.4 3.0) (end 74.4 18.0) (width 0.4) (layer "F.Cu") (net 2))
 (segment (start 74.4 18.0) (end 74.4 46.0) (width 0.4) (layer "F.Cu") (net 2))
 (segment (start 79.2 7.0) (end 79.2 21.0) (width 0.2) (layer "F.Cu") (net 6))
 (segment (start 79.2 21.0) (end 79.2 48.4) (width 0.2) (layer "F.Cu") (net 6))
 (segment (start 79.2 48.4) (end 79.2 63.5) (width 0.2) (layer "F.Cu") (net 6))
 (segment (start 73.2 2.0) (end 73.2 32.0) (width 0.4) (layer "F.Cu") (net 1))
 (segment (start 73.2 32.0) (end 73.2 60.0) (width 0.4) (layer "F.Cu") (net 1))
 (segment (start 82.8 9.0) (end 82.8 23.25) (width 0.2) (layer "F.Cu") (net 7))
 (segment (start 82.8 23.25) (end 82.8 36.2857) (width 0.2) (layer "F.Cu") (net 7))
 (segment (start 75.6 4.0) (end 75.6 18.75) (width 0.2) (layer "F.Cu") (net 3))
 (segment (start 75.6 18.75) (end 75.6 32.8571) (width 0.2) (layer "F.Cu") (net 3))
 (segment (start 80.4 21.75) (end 80.4 34.5714) (width 0.2) (layer "F.Cu") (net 9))
 (segment (start 80.4 34.5714) (end 80.4 49.6) (width 0.2) (layer "F.Cu") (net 9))
 (segment (start 80.4 49.6) (end 80.4 65.25) (width 0.2) (layer "F.Cu") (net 9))
 (segment (start 81.6 8.0) (end 81.6 22.5) (width 0.2) (layer "F.Cu") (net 11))
 (segment (start 81.6 22.5) (end 81.6 35.4286) (width 0.2) (layer "F.Cu") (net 11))
 (segment (start 78.0 6.0) (end 78.0 20.25) (width 0.2) (layer "F.Cu") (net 5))
 (segment (start 78.0 20.25) (end 78.0 47.2) (width 0.2) (layer "F.Cu") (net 5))
 (segment (start 78.0 47.2) (end 78.0 61.75) (width 0.2) (layer "F.Cu") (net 5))
 (segment (start 86.4 37.1429) (end 86.4 50.8) (width 0.2) (layer "F.Cu") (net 12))
 (segment (start 86.4 50.8) (end 86.4 67.0) (width 0.2) (layer "F.Cu") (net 12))
 (via (at 21.0475 19.5) (size 0.8) (drill 0.4) (layers "F.Cu" "B.Cu") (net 4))
 (via (at 76.8 19.5) (size 0.8) (drill 0.4) (layers "F.Cu" "B.Cu") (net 4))
 (via (at 22.9525 18.0) (size 0.8) (drill 0.4) (layers "F.Cu" "B.Cu") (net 2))
 (via (at 74.4 18.0) (size 0.8) (drill 0.4) (layers "F.Cu" "B.Cu") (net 2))
 (via (at 22.0 7.0) (size 0.8) (drill 0.4) (layers "F.Cu" "B.Cu") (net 6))
 (via (at 79.2 7.0) (size 0.8) (drill 0.4) (layers "F.Cu" "B.Cu") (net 6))
 (via (at 21.0475 33.7143) (size 0.8) (drill 0.4) (layers "F.Cu" "B.Cu") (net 4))
 (via (at 76.8 33.7143) (size 0.8) (drill 0.4) (layers "F.Cu" "B.Cu") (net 4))
 (via (at 22.9525 32.0) (size 0.8) (drill 0.4) (layers "F.Cu" "B.Cu") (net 1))
 (via (at 73.2 32.0) (size 0.8) (drill 0.4) (layers "F.Cu" "B.Cu") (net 1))
 (via (at 22.0 21.0) (size 0.8) (drill 0.4) (layers "F.Cu" "B.Cu") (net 6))
 (via (at 79.2 21.0) (size 0.8) (drill 0.4) (layers "F.Cu" "B.Cu") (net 6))
 (via (at 29.0475 19.5) (size 0.8) (drill 0.4) (layers "F.Cu" "B.Cu") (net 4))
 (via (at 76.8 19.5) (size 0.8) (drill 0.4) (layers "F.Cu" "B.Cu") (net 4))
 (via (at 30.9525 18.0) (size 0.8) (drill 0.4) (layers "F.Cu" "B.Cu") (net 2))
 (via (at 74.4 18.0) (size 0.8) (drill 0.4) (layers "F.Cu" "B.Cu") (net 2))
 (via (at 30.0 9.0) (size 0.8) (drill 0.4) (layers "F.Cu" "B.Cu") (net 7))
 (via (at 82.8 9.0) (size 0.8) (drill 0.4) (layers "F.Cu" "B.Cu") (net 7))
 (via (at 29.0475 33.7143) (size 0.8) (drill 0.4) (layers "F.Cu" "B.Cu") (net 4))
 (via (at 76.8 33.7143) (size 0.8) (drill 0.4) (layers "F.Cu" "B.Cu") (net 4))
 (via (at 30.9525 32.0) (size 0.8) (drill 0.4) (layers "F.Cu" "B.Cu") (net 1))
 (via (at 73.2 32.0) (size 0.8) (drill 0.4) (layers "F.Cu" "B.Cu") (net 1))
 (via (at 30.0 23.25) (size 0.8) (drill 0.4) (layers "F.Cu" "B.Cu") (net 7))
 (via (at 82.8 23.25) (size 0.8) (drill 0.4) (layers "F.Cu" "B.Cu") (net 7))
 (via (at 37.0475 19.5) (size 0.8) (drill 0.4) (layers "F.Cu" "B.Cu") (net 4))
 (via (at 76.8 19.5) (size 0.8) (drill 0.4) (layers "F.Cu" "B.Cu") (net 4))
 (via (at 38.9525 18.75) (size 0.8) (drill 0.4) (layers "F.Cu" "B.Cu") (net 3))
 (via (at 75.6 18.75) (size 0.8) (drill 0.4) (layers "F.Cu" "B.Cu") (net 3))
 (via (at 38.0 10.0) (size 0.8) (drill 0.4) (layers "F.Cu" "B.Cu") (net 8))
 (via (at 84.0 10.0) (size 0.8) (drill 0.4) (layers "F.Cu" "B.Cu") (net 8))
 (via (at 45.0475 19.5) (size 0.8) (drill 0.4) (layers "F.Cu" "B.Cu") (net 4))
 (via (at 76.8 19.5) (size 0.8) (drill 0.4) (layers "F.Cu" "B.Cu") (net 4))
 (via (at 46.9525 21.75) (size 0.8) (drill 0.4) (layers "F.Cu" "B.Cu") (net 9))
 (via (at 80.4 21.75) (size 0.8) (drill 0.4) (layers "F.Cu" "B.Cu") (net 9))
 (via (at 46.0 10.0) (size 0.8) (drill 0.4) (layers "F.Cu" "B.Cu") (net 8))
 (via (at 84.0 10.0) (size 0.8) (drill 0.4) (layers "F.Cu" "B.Cu") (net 8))
 (via (at 37.0475 36.2857) (size 0.8) (drill 0.4) (layers "F.Cu" "B.Cu") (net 7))
 (via (at 82.8 36.2857) (size 0.8) (drill 0.4) (layers "F.Cu" "B.Cu") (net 7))
 (via (at 38.9525 32.8571) (size 0.8) (drill 0.4) (layers "F.Cu" "B.Cu") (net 3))
 (via (at 75.6 32.8571) (size 0.8) (drill 0.4) (layers "F.Cu" "B.Cu") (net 3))
 (via (at 38.0 24.0) (size 0.8) (drill 0.4) (layers "F.Cu" "B.Cu") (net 10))
 (via (at 85.2 24.0) (size 0.8) (drill 0.4) (layers "F.Cu" "B.Cu") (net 10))
 (via (at 45.0475 36.2857) (size 0.8) (drill 0.4) (layers "F.Cu" "B.Cu") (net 7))
 (via (at 82.8 36.2857) (size 0.8) (drill 0.4) (layers "F.Cu" "B.Cu") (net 7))
 (via (at 46.9525 34.5714) (size 0.8) (drill 0.4) (layers "F.Cu" "B.Cu") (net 9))
 (via (at 80.4 34.5714) (size 0.8) (drill 0.4) (layers "F.Cu" "B.Cu") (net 9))
 (via (at 46.0 24.0) (size 0.8) (drill 0.4) (layers "F.Cu" "B.Cu") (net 10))
 (via (at 85.2 24.0) (size 0.8) (drill 0.4) (layers "F.Cu" "B.Cu") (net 10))
 (via (at 53.0475 21.75) (size 0.8) (drill 0.4) (layers "F.Cu" "B.Cu") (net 9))
 (via (at 80.4 21.75) (size 0.8) (drill 0.4) (layers "F.Cu" "B.Cu") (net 9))
 (via (at 54.9525 18.0) (size 0.8) (drill 0.4) (layers "F.Cu" "B.Cu") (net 2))
 (via (at 74.4 18.0) (size 0.8) (drill 0.4) (layers "F.Cu" "B.Cu") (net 2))
 (via (at 54.0 8.0) (size 0.8) (drill 0.4) (layers "F.Cu" "B.Cu") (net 11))
 (via (at 81.6 8.0) (size 0.8) (drill 0.4) (layers "F.Cu" "B.Cu") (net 11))
 (via (at 53.0475 34.5714) (size 0.8) (drill 0.4) (layers "F.Cu" "B.Cu") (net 9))
 (via (at 80.4 34.5714) (size 0.8) (drill 0.4) (layers "F.Cu" "B.Cu") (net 9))
 (via (at 54.9525 32.0) (size 0.8) (drill 0.4) (layers "F.Cu" "B.Cu") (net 1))
 (via (at 73.2 32.0) (size 0.8) (drill 0.4) (layers "F.Cu" "B.Cu") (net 1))
 (via (at 54.0 22.5) (size 0.8) (drill 0.4) (layers "F.Cu" "B.Cu") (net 11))
 (via (at 81.6 22.5) (size 0.8) (drill 0.4) (layers "F.Cu" "B.Cu") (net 11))
 (via (at 61.0475 22.5) (size 0.8) (drill 0.4) (layers "F.Cu" "B.Cu") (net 11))
 (via (at 81.6 22.5) (size 0.8) (drill 0.4) (layers "F.Cu" "B.Cu") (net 11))
 (via (at 62.9525 18.0) (size 0.8) (drill 0.4) (layers "F.Cu" "B.Cu") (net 2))
 (via (at 74.4 18.0) (size 0.8) (drill 0.4) (layers "F.Cu" "B.Cu") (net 2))
 (via (at 62.0 6.0) (size 0.8) (drill 0.4) (layers "F.Cu" "B.Cu") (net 5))
 (via (at 78.0 6.0) (size 0.8) (drill 0.4) (layers "F.Cu" "B.Cu") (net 5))
 (via (at 61.0475 35.4286) (size 0.8) (drill 0.4) (layers "F.Cu" "B.Cu") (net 11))
 (via (at 81.6 35.4286) (size 0.8) (drill 0.4) (layers "F.Cu" "B.Cu") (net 11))
 (via (at 62.9525 32.0) (size 0.8) (drill 0.4) (layers "F.Cu" "B.Cu") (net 1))
 (via (at 73.2 32.0) (size 0.8) (drill 0.4) (layers "F.Cu" "B.Cu") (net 1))
 (via (at 62.0 20.25) (size 0.8) (drill 0.4) (layers "F.Cu" "B.Cu") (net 5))
 (via (at 78.0 20.25) (size 0.8) (drill 0.4) (layers "F.Cu" "B.Cu") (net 5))
 (via (at 29.0475 48.4) (size 0.8) (drill 0.4) (layers "F.Cu" "B.Cu") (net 6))
 (via (at 79.2 48.4) (size 0.8) (drill 0.4) (layers "F.Cu" "B.Cu") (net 6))
 (via (at 30.9525 46.0) (size 0.8) (drill 0.4) (layers "F.Cu" "B.Cu") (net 2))
 (via (at 74.4 46.0) (size 0.8) (drill 0.4) (layers "F.Cu" "B.Cu") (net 2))
 (via (at 30.0 37.1429) (size 0.8) (drill 0.4) (layers "F.Cu" "B.Cu") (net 12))
 (via (at 86.4 37.1429) (size 0.8) (drill 0.4) (layers "F.Cu" "B.Cu") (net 12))
 (via (at 29.0475 63.5) (size 0.8) (drill 0.4) (layers "F.Cu" "B.Cu") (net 6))
 (via (at 79.2 63.5) (size 0.8) (drill 0.4) (layers "F.Cu" "B.Cu") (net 6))
 (via (at 30.9525 60.0) (size 0.8) (drill 0.4) (layers "F.Cu" "B.Cu") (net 1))
 (via (at 73.2 60.0) (size 0.8) (drill 0.4) (layers "F.Cu" "B.Cu") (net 1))
 (via (at 30.0 50.8) (size 0.8) (drill 0.4) (layers "F.Cu" "B.Cu") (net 12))
 (via (at 86.4 50.8) (size 0.8) (drill 0.4) (layers "F.Cu" "B.Cu") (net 12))
 (via (at 37.0475 48.4) (size 0.8) (drill 0.4) (layers "F.Cu" "B.Cu") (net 6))
 (via (at 79.2 48.4) (size 0.8) (drill 0.4) (layers "F.Cu" "B.Cu") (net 6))
 (via (at 38.9525 47.2) (size 0.8) (drill 0.4) (layers "F.Cu" "B.Cu") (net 5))
 (via (at 78.0 47.2) (size 0.8) (drill 0.4) (layers "F.Cu" "B.Cu") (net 5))
 (via (at 38.0 38.0) (size 0.8) (drill 0.4) (layers "F.Cu" "B.Cu") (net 13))
 (via (at 87.6 38.0) (size 0.8) (drill 0.4) (layers "F.Cu" "B.Cu") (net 13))
 (via (at 45.0475 48.4) (size 0.8) (drill 0.4) (layers "F.Cu" "B.Cu") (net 6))
 (via (at 79.2 48.4) (size 0.8) (drill 0.4) (layers "F.Cu" "B.Cu") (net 6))
 (via (at 46.9525 49.6) (size 0.8) (drill 0.4) (layers "F.Cu" "B.Cu") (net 9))
 (via (at 80.4 49.6) (size 0.8) (drill 0.4) (layers "F.Cu" "B.Cu") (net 9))
 (via (at 46.0 38.0) (size 0.8) (drill 0.4) (layers "F.Cu" "B.Cu") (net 13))
 (via (at 87.6 38.0) (size 0.8) (drill 0.4) (layers "F.Cu" "B.Cu") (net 13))
 (via (at 37.0475 67.0) (size 0.8) (drill 0.4) (layers "F.Cu" "B.Cu") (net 12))
 (via (at 86.4 67.0) (size 0.8) (drill 0.4) (layers "F.Cu" "B.Cu") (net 12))
 (via (at 38.9525 61.75) (size 0.8) (drill 0.4) (layers "F.Cu" "B.Cu") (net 5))
 (via (at 78.0 61.75) (size 0.8) (drill 0.4) (layers "F.Cu" "B.Cu") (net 5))
 (via (at 38.0 52.0) (size 0.8) (drill 0.4) (layers "F.Cu" "B.Cu") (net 14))
 (via (at 88.8 52.0) (size 0.8) (drill 0.4) (layers "F.Cu" "B.Cu") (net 14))
 (via (at 45.0475 67.0) (size 0.8) (drill 0.4) (layers "F.Cu" "B.Cu") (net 12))
 (via (at 86.4 67.0) (size 0.8) (drill 0.4) (layers "F.Cu" "B.Cu") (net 12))
 (via (at 46.9525 65.25) (size 0.8) (drill 0.4) (layers "F.Cu" "B.Cu") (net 9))
 (via (at 80.4 65.25) (size 0.8) (drill 0.4) (layers "F.Cu" "B.Cu") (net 9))
 (via (at 46.0 52.0) (size 0.8) (drill 0.4) (layers "F.Cu" "B.Cu") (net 14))
 (via (at 88.8 52.0) (size 0.8) (drill 0.4) (layers "F.Cu" "B.Cu") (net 14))
 (via (at 2.0 8.0) (size 0.8) (drill 0.4) (layers "F.Cu" "B.Cu") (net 1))
 (via (at 2.0 2.0) (size 0.8) (drill 0.4) (layers "F.Cu" "B.Cu") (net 1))
 (via (at 73.2 2.0) (size 0.8) (drill 0.4) (layers "F.Cu" "B.Cu") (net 1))
 (via (at 2.9 10.54) (size 0.8) (drill 0.4) (layers "F.Cu" "B.Cu") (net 2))
 (via (at 2.9 3.0) (size 0.8) (drill 0.4) (layers "F.Cu" "B.Cu") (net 2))
 (via (at 74.4 3.0) (size 0.8) (drill 0.4) (layers "F.Cu" "B.Cu") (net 2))
 (via (at 3.8 13.08) (size 0.8) (drill 0.4) (layers "F.Cu" "B.Cu") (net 3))
 (via (at 3.8 4.0) (size 0.8) (drill 0.4) (layers "F.Cu" "B.Cu") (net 3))
 (via (at 75.6 4.0) (size 0.8) (drill 0.4) (layers "F.Cu" "B.Cu") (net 3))
 (via (at 4.7 15.62) (size 0.8) (drill 0.4) (layers "F.Cu" "B.Cu") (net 4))
 (via (at 4.7 5.0) (size 0.8) (drill 0.4) (layers "F.Cu" "B.Cu") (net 4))
 (via (at 76.8 5.0) (size 0.8) (drill 0.4) (layers "F.Cu" "B.Cu") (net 4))
 (via (at 5.6 18.16) (size 0.8) (drill 0.4) (layers "F.Cu" "B.Cu") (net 5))
 (via (at 5.6 6.0) (size 0.8) (drill 0.4) (layers "F.Cu" "B.Cu") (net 5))
 (via (at 78.0 6.0) (size 0.8) (drill 0.4) (layers "F.Cu" "B.Cu") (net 5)))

